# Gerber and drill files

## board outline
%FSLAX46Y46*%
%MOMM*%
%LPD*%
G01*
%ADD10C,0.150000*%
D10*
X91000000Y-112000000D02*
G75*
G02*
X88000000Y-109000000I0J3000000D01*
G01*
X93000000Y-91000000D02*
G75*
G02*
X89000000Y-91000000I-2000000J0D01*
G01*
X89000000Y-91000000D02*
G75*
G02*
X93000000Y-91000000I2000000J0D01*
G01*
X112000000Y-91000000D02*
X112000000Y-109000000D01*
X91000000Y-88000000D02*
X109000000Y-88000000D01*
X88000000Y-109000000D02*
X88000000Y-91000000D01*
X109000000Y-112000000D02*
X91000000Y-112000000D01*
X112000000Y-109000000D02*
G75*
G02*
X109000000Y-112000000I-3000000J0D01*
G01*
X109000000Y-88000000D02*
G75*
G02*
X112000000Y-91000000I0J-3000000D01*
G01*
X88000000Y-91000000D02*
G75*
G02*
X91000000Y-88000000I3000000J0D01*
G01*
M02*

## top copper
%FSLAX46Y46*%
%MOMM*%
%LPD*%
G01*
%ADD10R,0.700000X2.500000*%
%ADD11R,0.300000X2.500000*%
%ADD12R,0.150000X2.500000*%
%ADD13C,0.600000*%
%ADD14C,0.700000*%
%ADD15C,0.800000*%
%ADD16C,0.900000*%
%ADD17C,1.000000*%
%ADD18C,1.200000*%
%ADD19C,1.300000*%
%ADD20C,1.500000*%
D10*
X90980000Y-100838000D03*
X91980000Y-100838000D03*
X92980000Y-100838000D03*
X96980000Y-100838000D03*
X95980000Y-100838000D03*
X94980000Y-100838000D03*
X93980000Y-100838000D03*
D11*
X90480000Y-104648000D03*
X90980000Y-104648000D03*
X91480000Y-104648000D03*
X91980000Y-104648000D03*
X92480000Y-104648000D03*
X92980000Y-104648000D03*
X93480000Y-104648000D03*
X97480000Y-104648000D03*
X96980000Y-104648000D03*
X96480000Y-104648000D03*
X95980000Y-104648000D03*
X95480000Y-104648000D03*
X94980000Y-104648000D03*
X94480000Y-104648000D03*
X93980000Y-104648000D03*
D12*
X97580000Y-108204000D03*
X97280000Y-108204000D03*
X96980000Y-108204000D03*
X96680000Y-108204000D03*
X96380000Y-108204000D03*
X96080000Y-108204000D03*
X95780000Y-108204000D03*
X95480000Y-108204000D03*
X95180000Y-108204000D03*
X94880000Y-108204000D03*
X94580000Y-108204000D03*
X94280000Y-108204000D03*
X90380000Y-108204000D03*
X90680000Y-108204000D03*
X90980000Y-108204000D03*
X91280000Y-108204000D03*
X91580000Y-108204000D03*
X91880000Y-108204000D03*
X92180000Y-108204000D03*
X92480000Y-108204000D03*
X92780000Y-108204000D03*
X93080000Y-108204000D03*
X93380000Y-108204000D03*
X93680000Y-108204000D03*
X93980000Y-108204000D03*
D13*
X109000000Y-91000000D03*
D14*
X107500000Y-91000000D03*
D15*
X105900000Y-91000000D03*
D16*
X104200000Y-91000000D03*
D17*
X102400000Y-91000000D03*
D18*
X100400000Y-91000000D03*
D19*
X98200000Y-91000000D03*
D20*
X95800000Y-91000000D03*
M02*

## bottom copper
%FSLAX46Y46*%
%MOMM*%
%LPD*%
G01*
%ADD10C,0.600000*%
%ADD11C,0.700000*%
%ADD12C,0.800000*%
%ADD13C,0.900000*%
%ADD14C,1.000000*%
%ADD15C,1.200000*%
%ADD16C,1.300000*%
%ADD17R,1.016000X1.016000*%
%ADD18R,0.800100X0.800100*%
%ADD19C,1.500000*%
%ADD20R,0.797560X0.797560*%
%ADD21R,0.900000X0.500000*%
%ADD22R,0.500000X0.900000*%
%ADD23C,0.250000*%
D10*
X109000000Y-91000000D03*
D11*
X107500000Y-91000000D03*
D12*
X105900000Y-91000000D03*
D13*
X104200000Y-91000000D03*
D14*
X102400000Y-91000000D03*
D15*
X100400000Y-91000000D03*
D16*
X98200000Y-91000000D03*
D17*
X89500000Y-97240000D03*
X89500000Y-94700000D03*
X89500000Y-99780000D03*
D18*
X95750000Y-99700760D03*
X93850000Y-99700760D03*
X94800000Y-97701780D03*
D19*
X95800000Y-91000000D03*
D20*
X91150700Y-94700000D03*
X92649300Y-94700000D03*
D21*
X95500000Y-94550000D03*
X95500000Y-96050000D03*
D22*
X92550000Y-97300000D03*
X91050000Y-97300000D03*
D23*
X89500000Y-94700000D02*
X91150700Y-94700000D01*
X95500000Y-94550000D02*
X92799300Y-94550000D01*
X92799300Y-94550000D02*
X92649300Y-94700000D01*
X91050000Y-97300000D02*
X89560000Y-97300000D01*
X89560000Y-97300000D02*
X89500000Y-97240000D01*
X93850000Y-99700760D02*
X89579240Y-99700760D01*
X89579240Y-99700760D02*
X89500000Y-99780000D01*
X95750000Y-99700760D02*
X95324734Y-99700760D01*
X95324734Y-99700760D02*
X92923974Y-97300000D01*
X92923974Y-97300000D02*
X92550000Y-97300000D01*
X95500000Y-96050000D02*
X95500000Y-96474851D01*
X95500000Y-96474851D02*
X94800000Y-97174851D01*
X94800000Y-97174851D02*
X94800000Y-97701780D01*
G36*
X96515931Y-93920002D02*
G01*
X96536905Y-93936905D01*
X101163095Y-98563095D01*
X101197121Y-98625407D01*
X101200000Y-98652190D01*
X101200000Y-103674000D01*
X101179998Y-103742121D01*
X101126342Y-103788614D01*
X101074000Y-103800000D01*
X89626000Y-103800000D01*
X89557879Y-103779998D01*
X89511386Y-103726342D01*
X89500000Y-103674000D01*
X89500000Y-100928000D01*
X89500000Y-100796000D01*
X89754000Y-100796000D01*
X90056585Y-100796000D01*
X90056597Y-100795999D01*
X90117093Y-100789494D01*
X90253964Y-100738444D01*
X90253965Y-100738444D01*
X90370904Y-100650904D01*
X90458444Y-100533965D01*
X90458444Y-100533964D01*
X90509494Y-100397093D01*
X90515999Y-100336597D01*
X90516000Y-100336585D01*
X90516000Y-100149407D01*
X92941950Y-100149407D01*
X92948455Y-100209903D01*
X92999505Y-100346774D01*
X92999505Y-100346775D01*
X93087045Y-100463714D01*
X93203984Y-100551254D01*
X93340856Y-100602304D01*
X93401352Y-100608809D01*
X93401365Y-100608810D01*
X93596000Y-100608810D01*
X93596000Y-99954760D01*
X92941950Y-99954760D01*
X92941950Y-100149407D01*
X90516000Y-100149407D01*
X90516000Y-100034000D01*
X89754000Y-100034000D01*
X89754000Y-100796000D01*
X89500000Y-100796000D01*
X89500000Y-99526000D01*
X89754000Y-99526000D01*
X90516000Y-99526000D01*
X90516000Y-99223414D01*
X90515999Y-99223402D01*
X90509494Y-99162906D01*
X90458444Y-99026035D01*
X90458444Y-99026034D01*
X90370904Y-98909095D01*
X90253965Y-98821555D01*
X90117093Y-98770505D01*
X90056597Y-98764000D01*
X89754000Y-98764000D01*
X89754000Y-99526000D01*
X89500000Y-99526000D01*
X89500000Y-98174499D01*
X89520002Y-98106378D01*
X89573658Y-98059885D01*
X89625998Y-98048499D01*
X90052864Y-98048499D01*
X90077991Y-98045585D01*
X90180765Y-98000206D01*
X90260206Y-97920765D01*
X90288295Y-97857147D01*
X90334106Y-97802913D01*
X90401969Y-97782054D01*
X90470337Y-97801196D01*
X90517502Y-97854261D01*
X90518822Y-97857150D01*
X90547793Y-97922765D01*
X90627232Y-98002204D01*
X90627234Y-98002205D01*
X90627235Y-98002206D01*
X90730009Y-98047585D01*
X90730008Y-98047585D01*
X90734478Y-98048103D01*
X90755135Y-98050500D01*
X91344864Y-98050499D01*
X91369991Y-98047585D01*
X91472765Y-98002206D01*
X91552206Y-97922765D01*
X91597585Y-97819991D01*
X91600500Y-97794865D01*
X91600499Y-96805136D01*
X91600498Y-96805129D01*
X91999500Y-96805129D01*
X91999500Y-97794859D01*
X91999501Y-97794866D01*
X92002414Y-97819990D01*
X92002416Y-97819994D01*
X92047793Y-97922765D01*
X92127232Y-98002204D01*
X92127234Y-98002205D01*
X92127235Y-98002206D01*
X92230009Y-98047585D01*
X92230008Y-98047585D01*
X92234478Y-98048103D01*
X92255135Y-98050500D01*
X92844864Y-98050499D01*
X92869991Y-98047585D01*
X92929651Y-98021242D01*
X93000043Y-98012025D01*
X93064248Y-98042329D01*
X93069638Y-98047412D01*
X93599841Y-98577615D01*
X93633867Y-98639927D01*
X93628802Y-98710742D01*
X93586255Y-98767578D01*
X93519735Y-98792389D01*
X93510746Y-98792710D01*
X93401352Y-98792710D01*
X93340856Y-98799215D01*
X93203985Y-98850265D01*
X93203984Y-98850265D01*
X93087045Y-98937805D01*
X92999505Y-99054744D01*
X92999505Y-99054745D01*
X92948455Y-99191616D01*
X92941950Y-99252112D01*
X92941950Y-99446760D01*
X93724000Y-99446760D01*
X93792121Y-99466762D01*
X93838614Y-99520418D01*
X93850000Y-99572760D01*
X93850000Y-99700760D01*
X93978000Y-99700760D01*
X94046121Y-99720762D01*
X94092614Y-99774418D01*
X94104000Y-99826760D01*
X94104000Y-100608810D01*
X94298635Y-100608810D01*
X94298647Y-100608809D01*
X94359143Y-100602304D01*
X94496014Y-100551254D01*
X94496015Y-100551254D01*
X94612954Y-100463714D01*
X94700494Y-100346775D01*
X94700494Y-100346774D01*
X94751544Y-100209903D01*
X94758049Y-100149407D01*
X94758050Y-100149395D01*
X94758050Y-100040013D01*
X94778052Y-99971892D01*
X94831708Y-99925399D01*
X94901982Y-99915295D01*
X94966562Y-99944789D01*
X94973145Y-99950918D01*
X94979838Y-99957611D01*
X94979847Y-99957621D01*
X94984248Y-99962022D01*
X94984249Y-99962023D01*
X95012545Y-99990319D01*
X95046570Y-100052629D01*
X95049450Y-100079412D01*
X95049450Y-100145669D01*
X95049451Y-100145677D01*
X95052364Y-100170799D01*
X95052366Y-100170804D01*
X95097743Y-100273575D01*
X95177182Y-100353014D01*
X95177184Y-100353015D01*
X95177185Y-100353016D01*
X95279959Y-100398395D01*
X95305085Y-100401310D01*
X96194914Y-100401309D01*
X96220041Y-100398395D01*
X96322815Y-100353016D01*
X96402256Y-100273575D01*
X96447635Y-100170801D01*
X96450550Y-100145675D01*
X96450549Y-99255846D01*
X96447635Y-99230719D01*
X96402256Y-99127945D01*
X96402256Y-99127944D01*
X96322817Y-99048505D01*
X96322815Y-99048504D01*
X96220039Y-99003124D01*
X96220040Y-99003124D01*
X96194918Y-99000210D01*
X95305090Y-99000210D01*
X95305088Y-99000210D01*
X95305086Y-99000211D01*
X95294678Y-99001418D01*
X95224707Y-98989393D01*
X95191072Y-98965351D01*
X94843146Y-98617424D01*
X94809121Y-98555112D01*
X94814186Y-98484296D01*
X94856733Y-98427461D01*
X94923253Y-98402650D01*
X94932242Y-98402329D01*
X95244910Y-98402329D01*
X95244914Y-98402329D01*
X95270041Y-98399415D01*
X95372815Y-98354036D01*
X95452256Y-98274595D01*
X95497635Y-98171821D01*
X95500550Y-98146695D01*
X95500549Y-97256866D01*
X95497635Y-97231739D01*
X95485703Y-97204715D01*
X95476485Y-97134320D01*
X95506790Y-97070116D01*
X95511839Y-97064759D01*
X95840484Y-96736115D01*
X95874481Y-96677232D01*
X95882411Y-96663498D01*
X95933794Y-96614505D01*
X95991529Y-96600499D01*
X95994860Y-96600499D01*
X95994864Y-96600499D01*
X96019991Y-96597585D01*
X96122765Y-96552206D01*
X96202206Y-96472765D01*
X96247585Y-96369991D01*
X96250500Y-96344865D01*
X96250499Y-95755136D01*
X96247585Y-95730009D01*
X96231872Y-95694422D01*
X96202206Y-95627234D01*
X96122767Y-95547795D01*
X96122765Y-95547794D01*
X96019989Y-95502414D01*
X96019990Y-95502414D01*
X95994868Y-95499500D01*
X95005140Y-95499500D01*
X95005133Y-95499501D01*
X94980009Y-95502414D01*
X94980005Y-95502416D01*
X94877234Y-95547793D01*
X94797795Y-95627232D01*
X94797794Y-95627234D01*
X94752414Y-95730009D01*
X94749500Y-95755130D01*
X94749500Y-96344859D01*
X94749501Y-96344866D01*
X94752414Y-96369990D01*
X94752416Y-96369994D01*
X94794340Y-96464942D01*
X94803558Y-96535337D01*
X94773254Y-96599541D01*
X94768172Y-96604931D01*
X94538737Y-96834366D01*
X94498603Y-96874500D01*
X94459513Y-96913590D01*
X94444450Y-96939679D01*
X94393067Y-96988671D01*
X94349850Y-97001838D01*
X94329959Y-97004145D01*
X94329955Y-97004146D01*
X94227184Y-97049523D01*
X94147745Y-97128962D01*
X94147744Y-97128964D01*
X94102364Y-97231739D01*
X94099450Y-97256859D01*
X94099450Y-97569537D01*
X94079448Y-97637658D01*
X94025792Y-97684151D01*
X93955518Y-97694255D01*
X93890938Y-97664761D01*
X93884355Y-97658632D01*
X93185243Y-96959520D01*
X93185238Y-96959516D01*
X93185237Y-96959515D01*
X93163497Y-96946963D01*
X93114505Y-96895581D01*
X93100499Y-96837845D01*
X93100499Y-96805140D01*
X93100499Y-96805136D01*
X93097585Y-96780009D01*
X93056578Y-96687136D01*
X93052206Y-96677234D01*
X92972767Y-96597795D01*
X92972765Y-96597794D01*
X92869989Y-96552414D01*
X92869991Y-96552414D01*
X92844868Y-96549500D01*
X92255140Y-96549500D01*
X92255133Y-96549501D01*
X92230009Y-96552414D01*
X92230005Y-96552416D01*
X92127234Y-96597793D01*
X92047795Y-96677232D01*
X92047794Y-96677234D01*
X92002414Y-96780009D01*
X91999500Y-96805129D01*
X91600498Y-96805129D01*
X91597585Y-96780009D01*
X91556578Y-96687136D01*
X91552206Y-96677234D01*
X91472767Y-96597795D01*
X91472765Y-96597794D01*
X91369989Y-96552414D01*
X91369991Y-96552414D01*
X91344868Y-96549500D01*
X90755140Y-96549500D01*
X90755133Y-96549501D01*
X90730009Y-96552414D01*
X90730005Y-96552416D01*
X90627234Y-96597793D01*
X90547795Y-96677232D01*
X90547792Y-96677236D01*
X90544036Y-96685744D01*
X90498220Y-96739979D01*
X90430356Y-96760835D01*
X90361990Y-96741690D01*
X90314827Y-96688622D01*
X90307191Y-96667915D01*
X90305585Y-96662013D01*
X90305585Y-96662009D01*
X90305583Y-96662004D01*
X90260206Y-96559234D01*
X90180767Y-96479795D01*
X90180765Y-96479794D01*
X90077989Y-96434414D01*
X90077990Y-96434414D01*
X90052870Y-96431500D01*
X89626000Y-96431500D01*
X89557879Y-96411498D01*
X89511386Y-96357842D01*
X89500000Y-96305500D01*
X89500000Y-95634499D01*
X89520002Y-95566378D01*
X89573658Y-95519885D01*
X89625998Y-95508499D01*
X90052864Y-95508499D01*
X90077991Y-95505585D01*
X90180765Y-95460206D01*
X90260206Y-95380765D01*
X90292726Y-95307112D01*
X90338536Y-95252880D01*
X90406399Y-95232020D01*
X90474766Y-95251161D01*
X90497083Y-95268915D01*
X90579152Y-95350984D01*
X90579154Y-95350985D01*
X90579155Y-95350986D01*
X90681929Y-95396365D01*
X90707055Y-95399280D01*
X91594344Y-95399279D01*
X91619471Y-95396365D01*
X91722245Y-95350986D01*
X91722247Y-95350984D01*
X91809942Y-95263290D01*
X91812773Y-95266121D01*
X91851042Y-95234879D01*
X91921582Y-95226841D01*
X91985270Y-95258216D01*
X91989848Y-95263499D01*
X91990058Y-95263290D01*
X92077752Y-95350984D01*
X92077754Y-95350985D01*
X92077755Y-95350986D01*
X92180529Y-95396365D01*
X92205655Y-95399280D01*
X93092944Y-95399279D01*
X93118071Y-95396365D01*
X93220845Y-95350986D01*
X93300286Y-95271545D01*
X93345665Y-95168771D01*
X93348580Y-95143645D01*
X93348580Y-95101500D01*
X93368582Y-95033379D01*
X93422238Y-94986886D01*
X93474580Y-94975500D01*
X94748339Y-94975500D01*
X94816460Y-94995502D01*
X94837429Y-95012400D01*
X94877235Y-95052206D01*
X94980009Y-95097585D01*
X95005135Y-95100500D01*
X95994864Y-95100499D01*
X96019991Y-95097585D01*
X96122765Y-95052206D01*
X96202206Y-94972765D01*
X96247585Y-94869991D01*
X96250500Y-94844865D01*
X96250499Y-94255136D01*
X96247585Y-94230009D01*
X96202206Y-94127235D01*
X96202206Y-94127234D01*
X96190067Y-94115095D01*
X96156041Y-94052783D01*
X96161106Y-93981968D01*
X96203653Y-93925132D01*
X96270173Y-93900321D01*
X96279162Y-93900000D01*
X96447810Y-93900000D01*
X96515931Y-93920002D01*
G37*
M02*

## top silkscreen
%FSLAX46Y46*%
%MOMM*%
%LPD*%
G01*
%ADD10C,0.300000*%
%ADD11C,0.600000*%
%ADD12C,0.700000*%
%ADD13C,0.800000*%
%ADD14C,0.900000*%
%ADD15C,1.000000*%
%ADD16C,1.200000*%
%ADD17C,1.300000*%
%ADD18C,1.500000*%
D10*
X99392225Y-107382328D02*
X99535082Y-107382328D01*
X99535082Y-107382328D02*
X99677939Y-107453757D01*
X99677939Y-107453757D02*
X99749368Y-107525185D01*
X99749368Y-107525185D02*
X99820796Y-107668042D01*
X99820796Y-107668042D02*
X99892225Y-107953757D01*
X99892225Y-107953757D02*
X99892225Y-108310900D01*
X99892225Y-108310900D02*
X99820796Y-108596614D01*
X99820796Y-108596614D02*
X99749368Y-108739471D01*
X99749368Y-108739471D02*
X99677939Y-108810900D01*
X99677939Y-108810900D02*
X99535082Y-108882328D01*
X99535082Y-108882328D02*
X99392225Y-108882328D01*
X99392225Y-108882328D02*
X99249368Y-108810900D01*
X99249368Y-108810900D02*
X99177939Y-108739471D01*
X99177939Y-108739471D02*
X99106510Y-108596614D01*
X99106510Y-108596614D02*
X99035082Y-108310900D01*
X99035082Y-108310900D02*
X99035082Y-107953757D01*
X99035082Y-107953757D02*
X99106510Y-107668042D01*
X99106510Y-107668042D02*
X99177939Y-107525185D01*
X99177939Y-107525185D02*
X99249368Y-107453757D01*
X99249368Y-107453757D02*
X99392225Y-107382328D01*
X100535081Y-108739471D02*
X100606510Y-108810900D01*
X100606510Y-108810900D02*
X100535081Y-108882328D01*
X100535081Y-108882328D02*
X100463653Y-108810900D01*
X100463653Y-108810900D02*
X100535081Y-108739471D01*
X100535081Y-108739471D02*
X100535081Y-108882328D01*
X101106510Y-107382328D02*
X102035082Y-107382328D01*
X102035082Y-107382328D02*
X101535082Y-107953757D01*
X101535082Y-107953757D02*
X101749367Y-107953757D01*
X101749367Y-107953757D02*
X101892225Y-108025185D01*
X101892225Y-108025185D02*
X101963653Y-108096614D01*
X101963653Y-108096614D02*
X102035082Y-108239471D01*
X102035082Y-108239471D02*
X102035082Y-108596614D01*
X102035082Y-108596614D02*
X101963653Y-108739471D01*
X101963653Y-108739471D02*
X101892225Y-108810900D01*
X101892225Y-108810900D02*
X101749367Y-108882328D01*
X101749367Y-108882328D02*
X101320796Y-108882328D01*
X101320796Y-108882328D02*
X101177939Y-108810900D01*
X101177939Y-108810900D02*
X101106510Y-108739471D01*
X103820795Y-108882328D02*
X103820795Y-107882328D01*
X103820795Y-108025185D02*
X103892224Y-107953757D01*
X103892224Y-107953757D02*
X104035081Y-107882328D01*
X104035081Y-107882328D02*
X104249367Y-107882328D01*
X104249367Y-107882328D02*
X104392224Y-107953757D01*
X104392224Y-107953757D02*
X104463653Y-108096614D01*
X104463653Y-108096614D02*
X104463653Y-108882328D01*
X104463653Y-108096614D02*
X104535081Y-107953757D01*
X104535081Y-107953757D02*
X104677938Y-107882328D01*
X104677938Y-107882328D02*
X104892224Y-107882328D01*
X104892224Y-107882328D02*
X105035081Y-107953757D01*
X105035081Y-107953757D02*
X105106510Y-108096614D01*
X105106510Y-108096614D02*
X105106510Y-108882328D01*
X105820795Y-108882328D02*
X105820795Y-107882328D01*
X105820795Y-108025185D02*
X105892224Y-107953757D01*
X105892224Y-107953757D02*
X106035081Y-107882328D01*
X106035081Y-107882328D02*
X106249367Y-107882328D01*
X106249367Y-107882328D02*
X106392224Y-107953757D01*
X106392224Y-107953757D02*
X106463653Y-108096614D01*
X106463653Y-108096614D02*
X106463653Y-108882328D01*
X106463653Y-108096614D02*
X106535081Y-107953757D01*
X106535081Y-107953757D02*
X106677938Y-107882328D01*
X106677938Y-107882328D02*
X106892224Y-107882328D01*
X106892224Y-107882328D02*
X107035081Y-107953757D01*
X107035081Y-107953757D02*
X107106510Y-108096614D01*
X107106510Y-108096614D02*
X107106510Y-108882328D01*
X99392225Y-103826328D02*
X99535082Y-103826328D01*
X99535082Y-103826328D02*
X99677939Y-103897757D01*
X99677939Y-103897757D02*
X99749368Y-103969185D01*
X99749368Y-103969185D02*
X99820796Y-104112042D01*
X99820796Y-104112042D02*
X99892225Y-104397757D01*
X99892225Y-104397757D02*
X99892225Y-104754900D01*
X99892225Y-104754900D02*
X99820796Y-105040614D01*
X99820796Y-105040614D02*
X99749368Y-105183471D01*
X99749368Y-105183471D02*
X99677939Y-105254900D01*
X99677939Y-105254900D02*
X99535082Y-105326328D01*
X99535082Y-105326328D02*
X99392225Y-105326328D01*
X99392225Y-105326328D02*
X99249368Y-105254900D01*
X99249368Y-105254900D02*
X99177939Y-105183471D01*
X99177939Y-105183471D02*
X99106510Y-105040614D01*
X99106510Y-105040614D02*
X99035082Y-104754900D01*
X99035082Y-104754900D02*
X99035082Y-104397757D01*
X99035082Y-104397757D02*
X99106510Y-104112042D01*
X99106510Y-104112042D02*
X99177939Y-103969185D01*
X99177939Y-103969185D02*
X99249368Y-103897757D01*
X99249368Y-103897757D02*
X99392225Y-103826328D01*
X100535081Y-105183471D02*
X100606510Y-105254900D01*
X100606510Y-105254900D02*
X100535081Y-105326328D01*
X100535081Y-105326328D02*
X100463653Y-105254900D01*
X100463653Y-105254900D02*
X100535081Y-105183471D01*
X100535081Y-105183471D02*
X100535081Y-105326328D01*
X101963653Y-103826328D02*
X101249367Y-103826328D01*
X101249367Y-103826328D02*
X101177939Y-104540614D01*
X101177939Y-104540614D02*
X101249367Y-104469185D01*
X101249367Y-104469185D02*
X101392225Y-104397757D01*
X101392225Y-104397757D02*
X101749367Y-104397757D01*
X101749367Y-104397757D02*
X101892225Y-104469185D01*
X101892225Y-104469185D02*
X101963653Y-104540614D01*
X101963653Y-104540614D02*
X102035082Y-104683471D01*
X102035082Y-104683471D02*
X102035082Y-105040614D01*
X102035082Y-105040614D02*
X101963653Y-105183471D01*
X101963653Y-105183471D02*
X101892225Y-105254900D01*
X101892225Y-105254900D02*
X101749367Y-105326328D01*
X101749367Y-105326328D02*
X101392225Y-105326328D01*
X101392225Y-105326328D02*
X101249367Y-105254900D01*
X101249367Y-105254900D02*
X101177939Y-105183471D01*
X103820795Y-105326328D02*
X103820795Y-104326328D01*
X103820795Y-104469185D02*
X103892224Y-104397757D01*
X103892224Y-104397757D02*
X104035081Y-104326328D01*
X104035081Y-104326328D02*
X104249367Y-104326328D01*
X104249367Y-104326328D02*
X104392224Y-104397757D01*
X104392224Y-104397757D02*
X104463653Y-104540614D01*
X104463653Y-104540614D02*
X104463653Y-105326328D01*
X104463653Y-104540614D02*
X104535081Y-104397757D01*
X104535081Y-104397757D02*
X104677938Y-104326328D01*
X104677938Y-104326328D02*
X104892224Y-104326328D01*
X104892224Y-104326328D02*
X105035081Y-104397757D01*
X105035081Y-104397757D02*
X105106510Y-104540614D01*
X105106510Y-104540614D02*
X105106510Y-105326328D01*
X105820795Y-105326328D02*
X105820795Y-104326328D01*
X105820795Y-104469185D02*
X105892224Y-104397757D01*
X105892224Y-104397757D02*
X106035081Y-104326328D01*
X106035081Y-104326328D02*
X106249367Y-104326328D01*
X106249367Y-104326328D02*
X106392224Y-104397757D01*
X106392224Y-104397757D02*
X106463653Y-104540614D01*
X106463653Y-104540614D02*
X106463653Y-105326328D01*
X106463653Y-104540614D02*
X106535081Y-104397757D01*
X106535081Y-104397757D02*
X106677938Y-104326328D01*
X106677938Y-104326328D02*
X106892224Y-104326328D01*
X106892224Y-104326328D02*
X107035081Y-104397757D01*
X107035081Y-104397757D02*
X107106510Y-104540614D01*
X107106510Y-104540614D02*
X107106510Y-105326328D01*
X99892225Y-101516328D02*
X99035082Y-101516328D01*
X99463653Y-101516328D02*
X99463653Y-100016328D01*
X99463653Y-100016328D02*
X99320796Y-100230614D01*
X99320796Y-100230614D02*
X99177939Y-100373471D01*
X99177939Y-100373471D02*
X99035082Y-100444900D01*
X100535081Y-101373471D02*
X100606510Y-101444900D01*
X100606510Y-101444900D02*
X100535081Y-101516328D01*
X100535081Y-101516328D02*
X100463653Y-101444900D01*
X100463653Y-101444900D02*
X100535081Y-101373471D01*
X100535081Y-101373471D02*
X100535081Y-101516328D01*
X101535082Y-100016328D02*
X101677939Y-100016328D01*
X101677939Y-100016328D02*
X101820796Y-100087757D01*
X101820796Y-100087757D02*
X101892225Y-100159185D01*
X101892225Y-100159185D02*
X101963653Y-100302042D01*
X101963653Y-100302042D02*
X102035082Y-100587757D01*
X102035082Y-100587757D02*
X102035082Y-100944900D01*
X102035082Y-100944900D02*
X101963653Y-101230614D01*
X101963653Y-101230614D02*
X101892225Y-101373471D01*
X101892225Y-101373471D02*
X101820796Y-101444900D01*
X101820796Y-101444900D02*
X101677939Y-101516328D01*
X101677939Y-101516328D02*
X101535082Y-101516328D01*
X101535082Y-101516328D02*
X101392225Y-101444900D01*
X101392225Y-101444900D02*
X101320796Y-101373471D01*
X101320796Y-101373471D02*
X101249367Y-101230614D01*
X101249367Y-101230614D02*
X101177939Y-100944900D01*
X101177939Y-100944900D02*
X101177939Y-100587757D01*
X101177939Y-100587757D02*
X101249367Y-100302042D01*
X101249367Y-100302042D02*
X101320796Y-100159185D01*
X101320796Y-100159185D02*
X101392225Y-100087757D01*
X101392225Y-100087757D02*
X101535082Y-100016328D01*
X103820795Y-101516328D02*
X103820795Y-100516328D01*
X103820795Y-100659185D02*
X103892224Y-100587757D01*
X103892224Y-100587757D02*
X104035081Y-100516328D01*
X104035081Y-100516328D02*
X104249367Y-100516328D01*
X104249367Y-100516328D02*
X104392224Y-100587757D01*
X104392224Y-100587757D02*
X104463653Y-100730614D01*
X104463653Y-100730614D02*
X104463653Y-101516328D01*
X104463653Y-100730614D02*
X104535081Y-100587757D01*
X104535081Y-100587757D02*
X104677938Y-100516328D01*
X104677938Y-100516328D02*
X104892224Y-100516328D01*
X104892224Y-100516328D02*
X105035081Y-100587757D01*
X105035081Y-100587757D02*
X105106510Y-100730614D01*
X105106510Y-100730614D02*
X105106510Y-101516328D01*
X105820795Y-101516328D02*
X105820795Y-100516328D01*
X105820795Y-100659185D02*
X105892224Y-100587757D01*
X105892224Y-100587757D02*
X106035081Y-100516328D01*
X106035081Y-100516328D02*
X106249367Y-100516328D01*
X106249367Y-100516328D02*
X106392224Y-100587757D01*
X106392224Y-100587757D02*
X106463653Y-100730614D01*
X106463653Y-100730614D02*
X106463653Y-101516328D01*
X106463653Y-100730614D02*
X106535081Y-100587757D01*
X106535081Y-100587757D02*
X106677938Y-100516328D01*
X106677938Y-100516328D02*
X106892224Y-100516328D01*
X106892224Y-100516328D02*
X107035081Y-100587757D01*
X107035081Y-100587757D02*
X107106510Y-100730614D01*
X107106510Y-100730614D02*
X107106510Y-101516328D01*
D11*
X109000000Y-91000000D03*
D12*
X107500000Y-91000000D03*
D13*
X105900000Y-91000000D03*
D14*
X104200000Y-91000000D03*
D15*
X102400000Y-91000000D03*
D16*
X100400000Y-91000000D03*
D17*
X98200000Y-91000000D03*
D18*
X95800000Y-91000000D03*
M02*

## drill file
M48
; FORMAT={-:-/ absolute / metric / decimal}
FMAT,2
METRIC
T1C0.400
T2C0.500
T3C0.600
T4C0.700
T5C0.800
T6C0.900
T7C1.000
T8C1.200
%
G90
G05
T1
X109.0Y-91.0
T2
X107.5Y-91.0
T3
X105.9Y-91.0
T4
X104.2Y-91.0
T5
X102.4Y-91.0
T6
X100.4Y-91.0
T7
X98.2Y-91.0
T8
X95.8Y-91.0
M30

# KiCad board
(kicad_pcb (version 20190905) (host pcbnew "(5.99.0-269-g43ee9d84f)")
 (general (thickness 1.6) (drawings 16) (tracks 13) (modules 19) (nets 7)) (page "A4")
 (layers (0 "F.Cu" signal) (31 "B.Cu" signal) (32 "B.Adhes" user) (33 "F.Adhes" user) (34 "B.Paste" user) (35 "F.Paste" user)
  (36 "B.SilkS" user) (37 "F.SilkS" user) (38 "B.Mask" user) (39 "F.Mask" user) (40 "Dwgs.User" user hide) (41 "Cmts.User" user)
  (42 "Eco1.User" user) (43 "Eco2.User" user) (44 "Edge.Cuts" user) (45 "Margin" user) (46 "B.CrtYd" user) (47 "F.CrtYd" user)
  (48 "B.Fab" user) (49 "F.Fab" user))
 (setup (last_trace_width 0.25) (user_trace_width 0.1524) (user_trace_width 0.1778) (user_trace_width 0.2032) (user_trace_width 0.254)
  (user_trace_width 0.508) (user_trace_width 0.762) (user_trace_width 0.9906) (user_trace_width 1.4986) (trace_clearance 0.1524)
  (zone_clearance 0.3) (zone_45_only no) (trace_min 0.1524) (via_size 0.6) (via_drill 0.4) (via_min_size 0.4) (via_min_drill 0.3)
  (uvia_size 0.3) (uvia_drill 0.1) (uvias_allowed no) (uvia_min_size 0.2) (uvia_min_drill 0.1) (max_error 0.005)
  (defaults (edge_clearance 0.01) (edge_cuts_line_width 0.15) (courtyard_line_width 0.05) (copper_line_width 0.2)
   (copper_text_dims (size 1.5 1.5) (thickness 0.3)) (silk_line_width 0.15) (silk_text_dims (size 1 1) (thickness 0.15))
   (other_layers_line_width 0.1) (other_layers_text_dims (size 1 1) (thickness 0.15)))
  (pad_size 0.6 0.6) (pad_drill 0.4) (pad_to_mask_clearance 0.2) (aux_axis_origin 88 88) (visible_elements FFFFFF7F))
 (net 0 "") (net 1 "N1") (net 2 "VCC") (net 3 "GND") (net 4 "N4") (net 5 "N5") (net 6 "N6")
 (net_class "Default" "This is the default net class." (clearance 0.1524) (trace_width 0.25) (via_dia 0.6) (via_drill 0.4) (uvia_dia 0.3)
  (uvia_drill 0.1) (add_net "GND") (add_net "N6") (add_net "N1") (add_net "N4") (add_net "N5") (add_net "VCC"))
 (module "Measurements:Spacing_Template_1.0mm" (layer "F.Cu") (at 93.98 100.838)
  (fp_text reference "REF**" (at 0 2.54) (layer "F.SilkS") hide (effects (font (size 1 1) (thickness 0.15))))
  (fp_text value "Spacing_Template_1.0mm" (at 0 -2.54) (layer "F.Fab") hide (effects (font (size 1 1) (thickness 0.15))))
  (pad "1" smd rect (at -3 0) (size 0.7 2.5) (layers "F.Cu" "F.Paste" "F.Mask"))
  (pad "1" smd rect (at -2 0) (size 0.7 2.5) (layers "F.Cu" "F.Paste" "F.Mask"))
  (pad "1" smd rect (at -1 0) (size 0.7 2.5) (layers "F.Cu" "F.Paste" "F.Mask"))
  (pad "1" smd rect (at 3 0) (size 0.7 2.5) (layers "F.Cu" "F.Paste" "F.Mask"))
  (pad "1" smd rect (at 2 0) (size 0.7 2.5) (layers "F.Cu" "F.Paste" "F.Mask"))
  (pad "1" smd rect (at 1 0) (size 0.7 2.5) (layers "F.Cu" "F.Paste" "F.Mask"))
  (pad "1" smd rect (at 0 0) (size 0.7 2.5) (layers "F.Cu" "F.Paste" "F.Mask")))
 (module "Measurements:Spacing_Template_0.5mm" (layer "F.Cu") (at 93.98 104.648)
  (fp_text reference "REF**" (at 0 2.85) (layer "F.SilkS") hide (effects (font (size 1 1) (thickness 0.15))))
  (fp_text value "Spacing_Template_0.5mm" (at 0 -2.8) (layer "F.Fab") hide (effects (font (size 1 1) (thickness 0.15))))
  (pad "1" smd rect (at -3.5 0) (size 0.3 2.5) (layers "F.Cu" "F.Paste" "F.Mask"))
  (pad "1" smd rect (at -3 0) (size 0.3 2.5) (layers "F.Cu" "F.Paste" "F.Mask"))
  (pad "1" smd rect (at -2.5 0) (size 0.3 2.5) (layers "F.Cu" "F.Paste" "F.Mask"))
  (pad "1" smd rect (at -2 0) (size 0.3 2.5) (layers "F.Cu" "F.Paste" "F.Mask"))
  (pad "1" smd rect (at -1.5 0) (size 0.3 2.5) (layers "F.Cu" "F.Paste" "F.Mask"))
  (pad "1" smd rect (at -1 0) (size 0.3 2.5) (layers "F.Cu" "F.Paste" "F.Mask"))
  (pad "1" smd rect (at -0.5 0) (size 0.3 2.5) (layers "F.Cu" "F.Paste" "F.Mask"))
  (pad "1" smd rect (at 3.5 0) (size 0.3 2.5) (layers "F.Cu" "F.Paste" "F.Mask"))
  (pad "1" smd rect (at 3 0) (size 0.3 2.5) (layers "F.Cu" "F.Paste" "F.Mask"))
  (pad "1" smd rect (at 2.5 0) (size 0.3 2.5) (layers "F.Cu" "F.Paste" "F.Mask"))
  (pad "1" smd rect (at 2 0) (size 0.3 2.5) (layers "F.Cu" "F.Paste" "F.Mask"))
  (pad "1" smd rect (at 1.5 0) (size 0.3 2.5) (layers "F.Cu" "F.Paste" "F.Mask"))
  (pad "1" smd rect (at 1 0) (size 0.3 2.5) (layers "F.Cu" "F.Paste" "F.Mask"))
  (pad "1" smd rect (at 0.5 0) (size 0.3 2.5) (layers "F.Cu" "F.Paste" "F.Mask"))
  (pad "1" smd rect (at 0 0) (size 0.3 2.5) (layers "F.Cu" "F.Paste" "F.Mask")))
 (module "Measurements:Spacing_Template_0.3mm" (layer "F.Cu") (at 93.98 108.204)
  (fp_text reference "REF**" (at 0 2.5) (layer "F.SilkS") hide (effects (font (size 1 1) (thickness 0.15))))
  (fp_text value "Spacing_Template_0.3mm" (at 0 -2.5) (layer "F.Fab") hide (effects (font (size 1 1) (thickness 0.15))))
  (pad "1" smd rect (at 3.6 0) (size 0.15 2.5) (layers "F.Cu" "F.Paste" "F.Mask"))
  (pad "1" smd rect (at 3.3 0) (size 0.15 2.5) (layers "F.Cu" "F.Paste" "F.Mask"))
  (pad "1" smd rect (at 3 0) (size 0.15 2.5) (layers "F.Cu" "F.Paste" "F.Mask"))
  (pad "1" smd rect (at 2.7 0) (size 0.15 2.5) (layers "F.Cu" "F.Paste" "F.Mask"))
  (pad "1" smd rect (at 2.4 0) (size 0.15 2.5) (layers "F.Cu" "F.Paste" "F.Mask"))
  (pad "1" smd rect (at 2.1 0) (size 0.15 2.5) (layers "F.Cu" "F.Paste" "F.Mask"))
  (pad "1" smd rect (at 1.8 0) (size 0.15 2.5) (layers "F.Cu" "F.Paste" "F.Mask"))
  (pad "1" smd rect (at 1.5 0) (size 0.15 2.5) (layers "F.Cu" "F.Paste" "F.Mask"))
  (pad "1" smd rect (at 1.2 0) (size 0.15 2.5) (layers "F.Cu" "F.Paste" "F.Mask"))
  (pad "1" smd rect (at 0.9 0) (size 0.15 2.5) (layers "F.Cu" "F.Paste" "F.Mask"))
  (pad "1" smd rect (at 0.6 0) (size 0.15 2.5) (layers "F.Cu" "F.Paste" "F.Mask"))
  (pad "1" smd rect (at 0.3 0) (size 0.15 2.5) (layers "F.Cu" "F.Paste" "F.Mask"))
  (pad "1" smd rect (at -3.6 0) (size 0.15 2.5) (layers "F.Cu" "F.Paste" "F.Mask"))
  (pad "1" smd rect (at -3.3 0) (size 0.15 2.5) (layers "F.Cu" "F.Paste" "F.Mask"))
  (pad "1" smd rect (at -3 0) (size 0.15 2.5) (layers "F.Cu" "F.Paste" "F.Mask"))
  (pad "1" smd rect (at -2.7 0) (size 0.15 2.5) (layers "F.Cu" "F.Paste" "F.Mask"))
  (pad "1" smd rect (at -2.4 0) (size 0.15 2.5) (layers "F.Cu" "F.Paste" "F.Mask"))
  (pad "1" smd rect (at -2.1 0) (size 0.15 2.5) (layers "F.Cu" "F.Paste" "F.Mask"))
  (pad "1" smd rect (at -1.8 0) (size 0.15 2.5) (layers "F.Cu" "F.Paste" "F.Mask"))
  (pad "1" smd rect (at -1.5 0) (size 0.15 2.5) (layers "F.Cu" "F.Paste" "F.Mask"))
  (pad "1" smd rect (at -1.2 0) (size 0.15 2.5) (layers "F.Cu" "F.Paste" "F.Mask"))
  (pad "1" smd rect (at -0.9 0) (size 0.15 2.5) (layers "F.Cu" "F.Paste" "F.Mask"))
  (pad "1" smd rect (at -0.6 0) (size 0.15 2.5) (layers "F.Cu" "F.Paste" "F.Mask"))
  (pad "1" smd rect (at -0.3 0) (size 0.15 2.5) (layers "F.Cu" "F.Paste" "F.Mask"))
  (pad "1" smd rect (at 0 0) (size 0.15 2.5) (layers "F.Cu" "F.Paste" "F.Mask")))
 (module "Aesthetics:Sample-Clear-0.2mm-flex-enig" (layer "B.Cu") (at 100.0252 102.5652 180)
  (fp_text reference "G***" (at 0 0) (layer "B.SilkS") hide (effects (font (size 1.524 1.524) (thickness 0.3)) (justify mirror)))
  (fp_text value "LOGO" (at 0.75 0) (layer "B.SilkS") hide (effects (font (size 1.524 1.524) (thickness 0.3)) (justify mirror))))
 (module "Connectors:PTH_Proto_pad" (layer "F.Cu") (at 109 91)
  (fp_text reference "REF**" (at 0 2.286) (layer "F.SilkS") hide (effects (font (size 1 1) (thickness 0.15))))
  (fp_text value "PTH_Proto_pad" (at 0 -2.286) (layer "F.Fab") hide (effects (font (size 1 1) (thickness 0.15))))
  (pad "1" thru_hole circle (at 0 0) (size 0.6 0.6) (drill 0.4) (layers *.Cu *.Mask "F.SilkS")))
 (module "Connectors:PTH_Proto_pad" (layer "F.Cu") (at 107.5 91)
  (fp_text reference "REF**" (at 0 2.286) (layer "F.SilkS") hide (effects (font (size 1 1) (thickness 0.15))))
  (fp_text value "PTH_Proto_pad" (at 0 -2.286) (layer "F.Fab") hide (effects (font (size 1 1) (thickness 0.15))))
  (pad "1" thru_hole circle (at 0 0) (size 0.7 0.7) (drill 0.5) (layers *.Cu *.Mask "F.SilkS")))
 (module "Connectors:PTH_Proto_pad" (layer "F.Cu") (at 105.9 91)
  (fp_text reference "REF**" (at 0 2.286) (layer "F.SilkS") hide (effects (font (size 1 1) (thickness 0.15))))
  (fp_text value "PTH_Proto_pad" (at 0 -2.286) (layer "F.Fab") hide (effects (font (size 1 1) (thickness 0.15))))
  (pad "1" thru_hole circle (at 0 0) (size 0.8 0.8) (drill 0.6) (layers *.Cu *.Mask "F.SilkS")))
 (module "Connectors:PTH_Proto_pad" (layer "F.Cu") (at 104.2 91)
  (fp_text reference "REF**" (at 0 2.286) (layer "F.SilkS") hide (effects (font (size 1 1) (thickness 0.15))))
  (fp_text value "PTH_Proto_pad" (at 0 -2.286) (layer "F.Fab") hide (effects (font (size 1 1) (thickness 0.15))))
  (pad "1" thru_hole circle (at 0 0) (size 0.9 0.9) (drill 0.7) (layers *.Cu *.Mask "F.SilkS")))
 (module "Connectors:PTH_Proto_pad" (layer "F.Cu") (at 102.4 91)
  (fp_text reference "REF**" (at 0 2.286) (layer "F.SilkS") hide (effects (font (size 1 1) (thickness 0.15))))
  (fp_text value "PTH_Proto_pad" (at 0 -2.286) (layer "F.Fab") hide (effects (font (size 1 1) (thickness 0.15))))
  (pad "1" thru_hole circle (at 0 0) (size 1 1) (drill 0.8) (layers *.Cu *.Mask "F.SilkS")))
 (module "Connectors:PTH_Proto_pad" (layer "F.Cu") (at 100.4 91)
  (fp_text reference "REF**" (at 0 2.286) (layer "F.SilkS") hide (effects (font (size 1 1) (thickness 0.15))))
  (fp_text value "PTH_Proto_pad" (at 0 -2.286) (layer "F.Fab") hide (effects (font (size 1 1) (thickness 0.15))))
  (pad "1" thru_hole circle (at 0 0) (size 1.2 1.2) (drill 0.9) (layers *.Cu *.Mask "F.SilkS")))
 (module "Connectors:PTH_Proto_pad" (layer "F.Cu") (at 98.2 91)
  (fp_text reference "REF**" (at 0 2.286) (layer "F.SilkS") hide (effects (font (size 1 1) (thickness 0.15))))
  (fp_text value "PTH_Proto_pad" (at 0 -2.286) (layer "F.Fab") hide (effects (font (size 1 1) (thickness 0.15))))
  (pad "1" thru_hole circle (at 0 0) (size 1.3 1.3) (drill 1) (layers *.Cu *.Mask "F.SilkS")))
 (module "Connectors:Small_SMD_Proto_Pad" (layer "B.Cu") (at 89.5 97.24)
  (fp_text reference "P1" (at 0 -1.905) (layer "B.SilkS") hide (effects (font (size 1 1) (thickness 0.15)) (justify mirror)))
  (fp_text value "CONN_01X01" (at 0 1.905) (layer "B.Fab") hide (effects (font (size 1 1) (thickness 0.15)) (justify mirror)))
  (pad "1" smd rect (at 0 0) (size 1.016 1.016) (layers "B.Cu" "B.Paste" "B.Mask") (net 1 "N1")))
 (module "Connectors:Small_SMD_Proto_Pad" (layer "B.Cu") (at 89.5 94.7)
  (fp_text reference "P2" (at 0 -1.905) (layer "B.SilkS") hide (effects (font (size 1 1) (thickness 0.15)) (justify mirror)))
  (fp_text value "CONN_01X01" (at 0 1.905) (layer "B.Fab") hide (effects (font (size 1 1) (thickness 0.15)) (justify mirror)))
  (pad "1" smd rect (at 0 0) (size 1.016 1.016) (layers "B.Cu" "B.Paste" "B.Mask") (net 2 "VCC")))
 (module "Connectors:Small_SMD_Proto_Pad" (layer "B.Cu") (at 89.5 99.78)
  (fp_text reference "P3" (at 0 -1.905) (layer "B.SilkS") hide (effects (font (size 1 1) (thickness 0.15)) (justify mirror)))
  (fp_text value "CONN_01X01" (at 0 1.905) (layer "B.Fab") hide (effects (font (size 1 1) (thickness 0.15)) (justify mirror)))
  (pad "1" smd rect (at 0 0) (size 1.016 1.016) (layers "B.Cu" "B.Paste" "B.Mask") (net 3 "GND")))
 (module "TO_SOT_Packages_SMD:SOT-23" (layer "B.Cu") (at 94.8 98.7 180)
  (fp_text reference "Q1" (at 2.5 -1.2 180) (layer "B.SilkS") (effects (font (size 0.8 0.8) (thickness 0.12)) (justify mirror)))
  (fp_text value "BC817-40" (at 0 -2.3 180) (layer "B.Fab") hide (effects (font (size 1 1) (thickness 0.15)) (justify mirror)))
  (pad "1" smd rect (at -0.95 -1.00076 180) (size 0.8001 0.8001) (layers "B.Cu" "B.Paste" "B.Mask") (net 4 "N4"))
  (pad "2" smd rect (at 0.95 -1.00076 180) (size 0.8001 0.8001) (layers "B.Cu" "B.Paste" "B.Mask") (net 3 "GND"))
  (pad "3" smd rect (at 0 0.99822 180) (size 0.8001 0.8001) (layers "B.Cu" "B.Paste" "B.Mask") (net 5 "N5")))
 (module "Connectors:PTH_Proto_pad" (layer "F.Cu") (at 95.8 91)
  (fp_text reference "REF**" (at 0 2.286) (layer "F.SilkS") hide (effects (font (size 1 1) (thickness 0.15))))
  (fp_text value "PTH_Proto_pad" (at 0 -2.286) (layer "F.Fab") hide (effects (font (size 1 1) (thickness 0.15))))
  (pad "1" thru_hole circle (at 0 0) (size 1.5 1.5) (drill 1.2) (layers *.Cu *.Mask "F.SilkS")))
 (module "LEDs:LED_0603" (layer "B.Cu") (at 91.9 94.7 180)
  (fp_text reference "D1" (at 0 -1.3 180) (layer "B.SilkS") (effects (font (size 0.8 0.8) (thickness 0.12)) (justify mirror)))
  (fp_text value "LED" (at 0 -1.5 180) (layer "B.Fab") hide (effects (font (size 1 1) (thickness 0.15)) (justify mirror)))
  (pad "2" smd rect (at 0.7493 0) (size 0.79756 0.79756) (layers "B.Cu" "B.Paste" "B.Mask") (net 2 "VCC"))
  (pad "1" smd rect (at -0.7493 0) (size 0.79756 0.79756) (layers "B.Cu" "B.Paste" "B.Mask") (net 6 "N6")))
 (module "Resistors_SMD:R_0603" (layer "B.Cu") (at 95.5 95.3 -90)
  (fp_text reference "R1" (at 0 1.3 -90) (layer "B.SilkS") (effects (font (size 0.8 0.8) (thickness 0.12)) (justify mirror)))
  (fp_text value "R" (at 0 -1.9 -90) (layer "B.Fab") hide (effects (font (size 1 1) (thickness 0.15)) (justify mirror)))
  (pad "1" smd rect (at -0.75 0 270) (size 0.5 0.9) (layers "B.Cu" "B.Paste" "B.Mask") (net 6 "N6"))
  (pad "2" smd rect (at 0.75 0 270) (size 0.5 0.9) (layers "B.Cu" "B.Paste" "B.Mask") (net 5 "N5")))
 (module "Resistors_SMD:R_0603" (layer "B.Cu") (at 91.8 97.3 180)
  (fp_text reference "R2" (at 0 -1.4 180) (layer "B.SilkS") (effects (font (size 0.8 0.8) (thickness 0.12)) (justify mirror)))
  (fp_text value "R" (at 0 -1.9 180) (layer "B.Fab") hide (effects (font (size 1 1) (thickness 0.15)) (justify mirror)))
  (pad "1" smd rect (at -0.75 0 180) (size 0.5 0.9) (layers "B.Cu" "B.Paste" "B.Mask") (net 4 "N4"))
  (pad "2" smd rect (at 0.75 0 180) (size 0.5 0.9) (layers "B.Cu" "B.Paste" "B.Mask") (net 1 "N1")))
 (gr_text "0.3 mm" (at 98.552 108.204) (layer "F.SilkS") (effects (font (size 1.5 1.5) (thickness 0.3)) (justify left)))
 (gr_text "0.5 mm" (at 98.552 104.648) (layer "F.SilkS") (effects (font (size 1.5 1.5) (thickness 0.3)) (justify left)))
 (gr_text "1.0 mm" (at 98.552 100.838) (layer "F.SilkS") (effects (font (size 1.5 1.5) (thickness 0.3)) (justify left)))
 (gr_arc (start 91 109) (end 91 112) (angle 90) (layer "Edge.Cuts") (width 0.15))
 (gr_circle (center 91 91) (end 93 91) (layer "Edge.Cuts") (width 0.15))
 (gr_line (start 112 91) (end 112 109) (layer "Edge.Cuts") (width 0.15))
 (gr_line (start 91 88) (end 109 88) (layer "Edge.Cuts") (width 0.15))
 (gr_line (start 88 109) (end 88 91) (layer "Edge.Cuts") (width 0.15))
 (gr_line (start 109 112) (end 91 112) (layer "Edge.Cuts") (width 0.15))
 (gr_arc (start 109 109) (end 112 109) (angle 90) (layer "Edge.Cuts") (width 0.15))
 (gr_arc (start 109 91) (end 109 88) (angle 90) (layer "Edge.Cuts") (width 0.15))
 (gr_arc (start 91 91) (end 88 91) (angle 90) (layer "Edge.Cuts") (width 0.15))
 (segment (start 89.5 94.7) (end 91.1507 94.7) (width 0.25) (layer "B.Cu") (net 2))
 (segment (start 95.5 94.55) (end 92.7993 94.55) (width 0.25) (layer "B.Cu") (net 6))
 (segment (start 92.7993 94.55) (end 92.6493 94.7) (width 0.25) (layer "B.Cu") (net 6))
 (segment (start 91.05 97.3) (end 89.56 97.3) (width 0.25) (layer "B.Cu") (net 1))
 (segment (start 89.56 97.3) (end 89.5 97.24) (width 0.25) (layer "B.Cu") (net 1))
 (segment (start 93.85 99.70076) (end 89.57924 99.70076) (width 0.25) (layer "B.Cu") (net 3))
 (segment (start 89.57924 99.70076) (end 89.5 99.78) (width 0.25) (layer "B.Cu") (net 3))
 (segment (start 95.75 99.70076) (end 95.324734 99.70076) (width 0.25) (layer "B.Cu") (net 4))
 (segment (start 95.324734 99.70076) (end 92.923974 97.3) (width 0.25) (layer "B.Cu") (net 4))
 (segment (start 92.923974 97.3) (end 92.55 97.3) (width 0.25) (layer "B.Cu") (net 4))
 (segment (start 95.5 96.05) (end 95.5 96.474851) (width 0.25) (layer "B.Cu") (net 5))
 (segment (start 95.5 96.474851) (end 94.8 97.174851) (width 0.25) (layer "B.Cu") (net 5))
 (segment (start 94.8 97.174851) (end 94.8 97.70178) (width 0.25) (layer "B.Cu") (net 5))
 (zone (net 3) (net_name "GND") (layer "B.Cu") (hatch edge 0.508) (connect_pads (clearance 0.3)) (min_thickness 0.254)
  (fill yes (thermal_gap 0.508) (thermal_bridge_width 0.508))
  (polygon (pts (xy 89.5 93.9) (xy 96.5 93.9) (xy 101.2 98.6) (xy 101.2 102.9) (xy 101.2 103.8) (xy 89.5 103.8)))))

